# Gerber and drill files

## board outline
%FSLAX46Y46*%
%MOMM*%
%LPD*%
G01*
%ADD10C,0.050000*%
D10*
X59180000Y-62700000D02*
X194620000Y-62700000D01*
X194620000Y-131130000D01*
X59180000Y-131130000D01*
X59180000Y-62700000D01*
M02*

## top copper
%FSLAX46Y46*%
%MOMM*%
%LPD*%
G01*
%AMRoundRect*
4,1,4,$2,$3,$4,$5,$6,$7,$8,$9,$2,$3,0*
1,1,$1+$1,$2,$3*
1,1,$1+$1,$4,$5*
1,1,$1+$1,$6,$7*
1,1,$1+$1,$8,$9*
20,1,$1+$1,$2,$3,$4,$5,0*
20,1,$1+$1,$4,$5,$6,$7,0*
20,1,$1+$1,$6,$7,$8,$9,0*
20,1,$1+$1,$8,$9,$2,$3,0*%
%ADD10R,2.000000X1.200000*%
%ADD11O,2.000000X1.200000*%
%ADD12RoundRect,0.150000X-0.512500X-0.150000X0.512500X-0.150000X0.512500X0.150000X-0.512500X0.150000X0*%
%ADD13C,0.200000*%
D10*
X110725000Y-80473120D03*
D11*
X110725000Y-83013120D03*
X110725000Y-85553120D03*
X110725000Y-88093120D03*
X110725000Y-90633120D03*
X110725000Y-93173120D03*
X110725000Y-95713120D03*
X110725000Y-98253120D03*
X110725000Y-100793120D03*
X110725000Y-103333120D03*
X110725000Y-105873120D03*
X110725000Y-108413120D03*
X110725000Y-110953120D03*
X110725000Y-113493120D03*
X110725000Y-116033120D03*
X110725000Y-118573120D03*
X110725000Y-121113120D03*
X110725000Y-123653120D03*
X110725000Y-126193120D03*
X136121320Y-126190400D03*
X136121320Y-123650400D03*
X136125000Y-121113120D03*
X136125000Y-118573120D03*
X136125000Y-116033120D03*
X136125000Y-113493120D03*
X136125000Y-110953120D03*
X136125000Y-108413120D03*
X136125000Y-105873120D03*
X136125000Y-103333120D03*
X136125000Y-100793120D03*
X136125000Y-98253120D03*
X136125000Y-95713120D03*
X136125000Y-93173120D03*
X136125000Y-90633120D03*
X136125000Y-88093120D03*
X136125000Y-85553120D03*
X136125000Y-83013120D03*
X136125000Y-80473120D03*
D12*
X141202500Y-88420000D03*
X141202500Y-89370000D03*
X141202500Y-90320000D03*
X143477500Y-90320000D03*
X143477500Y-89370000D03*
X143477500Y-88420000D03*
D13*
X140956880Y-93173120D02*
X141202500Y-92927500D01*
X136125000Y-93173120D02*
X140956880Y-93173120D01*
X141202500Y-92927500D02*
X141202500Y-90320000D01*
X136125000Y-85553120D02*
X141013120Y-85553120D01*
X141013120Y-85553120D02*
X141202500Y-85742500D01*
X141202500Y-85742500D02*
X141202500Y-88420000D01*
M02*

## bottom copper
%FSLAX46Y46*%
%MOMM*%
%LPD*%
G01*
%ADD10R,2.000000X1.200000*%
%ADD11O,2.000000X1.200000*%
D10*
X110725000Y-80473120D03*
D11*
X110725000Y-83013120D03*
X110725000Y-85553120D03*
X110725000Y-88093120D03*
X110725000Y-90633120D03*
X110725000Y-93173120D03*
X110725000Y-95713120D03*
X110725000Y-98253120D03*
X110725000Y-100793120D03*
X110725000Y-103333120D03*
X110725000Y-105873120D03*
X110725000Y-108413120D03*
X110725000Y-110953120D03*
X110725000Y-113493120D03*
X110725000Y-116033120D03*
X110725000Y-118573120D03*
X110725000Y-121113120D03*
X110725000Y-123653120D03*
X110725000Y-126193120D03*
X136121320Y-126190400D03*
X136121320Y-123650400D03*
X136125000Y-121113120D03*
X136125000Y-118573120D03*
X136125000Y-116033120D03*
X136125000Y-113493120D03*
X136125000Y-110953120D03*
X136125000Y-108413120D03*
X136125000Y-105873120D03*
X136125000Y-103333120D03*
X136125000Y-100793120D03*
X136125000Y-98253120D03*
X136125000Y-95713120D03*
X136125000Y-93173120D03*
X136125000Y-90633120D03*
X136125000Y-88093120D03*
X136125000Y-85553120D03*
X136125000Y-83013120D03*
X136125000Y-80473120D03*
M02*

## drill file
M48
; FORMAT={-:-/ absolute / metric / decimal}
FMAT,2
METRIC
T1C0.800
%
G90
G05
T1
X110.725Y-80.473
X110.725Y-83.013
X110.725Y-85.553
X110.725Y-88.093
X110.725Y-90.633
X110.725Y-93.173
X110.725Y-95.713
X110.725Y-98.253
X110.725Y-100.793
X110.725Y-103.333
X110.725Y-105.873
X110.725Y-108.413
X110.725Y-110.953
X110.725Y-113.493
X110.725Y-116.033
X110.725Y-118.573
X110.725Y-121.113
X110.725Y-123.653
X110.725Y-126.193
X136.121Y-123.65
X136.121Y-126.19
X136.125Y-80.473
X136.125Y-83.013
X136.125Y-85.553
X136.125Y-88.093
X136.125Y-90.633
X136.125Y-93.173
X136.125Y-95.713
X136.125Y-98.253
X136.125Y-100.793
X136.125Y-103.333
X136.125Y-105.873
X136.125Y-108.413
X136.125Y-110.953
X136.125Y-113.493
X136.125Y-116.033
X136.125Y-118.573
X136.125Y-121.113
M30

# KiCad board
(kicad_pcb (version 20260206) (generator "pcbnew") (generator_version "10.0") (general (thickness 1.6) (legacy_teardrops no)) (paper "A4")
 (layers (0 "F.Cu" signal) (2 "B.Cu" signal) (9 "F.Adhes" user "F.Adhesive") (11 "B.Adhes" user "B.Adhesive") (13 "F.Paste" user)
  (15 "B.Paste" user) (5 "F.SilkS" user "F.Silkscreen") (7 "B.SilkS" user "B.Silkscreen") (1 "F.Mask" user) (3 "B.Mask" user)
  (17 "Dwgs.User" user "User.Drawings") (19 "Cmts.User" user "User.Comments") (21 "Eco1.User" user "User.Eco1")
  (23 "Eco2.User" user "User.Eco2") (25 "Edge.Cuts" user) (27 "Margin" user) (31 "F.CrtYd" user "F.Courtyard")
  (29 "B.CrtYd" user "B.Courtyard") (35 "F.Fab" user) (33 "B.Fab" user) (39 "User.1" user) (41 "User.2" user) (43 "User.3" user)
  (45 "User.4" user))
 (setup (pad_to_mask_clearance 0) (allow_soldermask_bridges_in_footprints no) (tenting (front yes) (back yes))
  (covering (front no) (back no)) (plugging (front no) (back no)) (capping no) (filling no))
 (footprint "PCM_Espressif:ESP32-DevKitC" (layer "F.Cu") (at 110.725 80.47312)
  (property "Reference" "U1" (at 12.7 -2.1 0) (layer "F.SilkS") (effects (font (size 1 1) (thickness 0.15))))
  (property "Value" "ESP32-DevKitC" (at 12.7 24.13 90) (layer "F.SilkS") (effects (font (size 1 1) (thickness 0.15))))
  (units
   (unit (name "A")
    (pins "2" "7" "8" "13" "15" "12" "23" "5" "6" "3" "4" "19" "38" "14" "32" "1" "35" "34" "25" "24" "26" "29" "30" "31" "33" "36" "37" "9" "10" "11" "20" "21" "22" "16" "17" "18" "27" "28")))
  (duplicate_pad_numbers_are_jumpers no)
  (pad "1" thru_hole rect (at 0 0 270) (size 1.2 2) (drill 0.8) (layers "*.Cu" "*.Mask") (remove_unused_layers no) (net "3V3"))
  (pad "2" thru_hole oval (at 0 2.54 270) (size 1.2 2) (drill 0.8) (layers "*.Cu" "*.Mask") (remove_unused_layers no)
   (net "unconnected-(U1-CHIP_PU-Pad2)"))
  (pad "3" thru_hole oval (at 0 5.08 270) (size 1.2 2) (drill 0.8) (layers "*.Cu" "*.Mask") (remove_unused_layers no)
   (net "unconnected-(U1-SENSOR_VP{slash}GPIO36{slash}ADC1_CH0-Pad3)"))
  (pad "4" thru_hole oval (at 0 7.62 270) (size 1.2 2) (drill 0.8) (layers "*.Cu" "*.Mask") (remove_unused_layers no)
   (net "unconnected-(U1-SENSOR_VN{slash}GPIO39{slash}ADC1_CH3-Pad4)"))
  (pad "5" thru_hole oval (at 0 10.16 270) (size 1.2 2) (drill 0.8) (layers "*.Cu" "*.Mask") (remove_unused_layers no)
   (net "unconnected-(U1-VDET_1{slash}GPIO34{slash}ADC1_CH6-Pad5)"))
  (pad "6" thru_hole oval (at 0 12.7 270) (size 1.2 2) (drill 0.8) (layers "*.Cu" "*.Mask") (remove_unused_layers no)
   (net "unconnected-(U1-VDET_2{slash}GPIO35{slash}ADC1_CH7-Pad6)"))
  (pad "7" thru_hole oval (at 0 15.24 270) (size 1.2 2) (drill 0.8) (layers "*.Cu" "*.Mask") (remove_unused_layers no)
   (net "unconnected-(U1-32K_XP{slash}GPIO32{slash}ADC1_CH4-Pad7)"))
  (pad "8" thru_hole oval (at 0 17.78 270) (size 1.2 2) (drill 0.8) (layers "*.Cu" "*.Mask") (remove_unused_layers no)
   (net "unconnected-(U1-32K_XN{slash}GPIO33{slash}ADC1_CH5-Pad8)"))
  (pad "9" thru_hole oval (at 0 20.32 270) (size 1.2 2) (drill 0.8) (layers "*.Cu" "*.Mask") (remove_unused_layers no) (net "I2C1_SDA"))
  (pad "10" thru_hole oval (at 0 22.86 270) (size 1.2 2) (drill 0.8) (layers "*.Cu" "*.Mask") (remove_unused_layers no) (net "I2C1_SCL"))
  (pad "11" thru_hole oval (at 0 25.4 270) (size 1.2 2) (drill 0.8) (layers "*.Cu" "*.Mask") (remove_unused_layers no)
   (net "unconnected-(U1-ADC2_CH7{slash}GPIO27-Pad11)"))
  (pad "12" thru_hole oval (at 0 27.94 270) (size 1.2 2) (drill 0.8) (layers "*.Cu" "*.Mask") (remove_unused_layers no)
   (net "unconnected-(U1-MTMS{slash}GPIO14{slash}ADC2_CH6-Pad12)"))
  (pad "13" thru_hole oval (at 0 30.48 270) (size 1.2 2) (drill 0.8) (layers "*.Cu" "*.Mask") (remove_unused_layers no)
   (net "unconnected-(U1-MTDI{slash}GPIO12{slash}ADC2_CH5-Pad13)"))
  (pad "14" thru_hole oval (at 0 33.02 270) (size 1.2 2) (drill 0.8) (layers "*.Cu" "*.Mask") (remove_unused_layers no) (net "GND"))
  (pad "15" thru_hole oval (at 0 35.56 270) (size 1.2 2) (drill 0.8) (layers "*.Cu" "*.Mask") (remove_unused_layers no)
   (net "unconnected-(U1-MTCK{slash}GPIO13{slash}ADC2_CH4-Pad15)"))
  (pad "16" thru_hole oval (at 0 38.1 270) (size 1.2 2) (drill 0.8) (layers "*.Cu" "*.Mask") (remove_unused_layers no)
   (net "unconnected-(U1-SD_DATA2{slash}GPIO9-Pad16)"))
  (pad "17" thru_hole oval (at 0 40.64 270) (size 1.2 2) (drill 0.8) (layers "*.Cu" "*.Mask") (remove_unused_layers no)
   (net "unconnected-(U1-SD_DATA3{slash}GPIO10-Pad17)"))
  (pad "18" thru_hole oval (at 0 43.18 270) (size 1.2 2) (drill 0.8) (layers "*.Cu" "*.Mask") (remove_unused_layers no)
   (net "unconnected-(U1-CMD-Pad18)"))
  (pad "19" thru_hole oval (at 0 45.72 270) (size 1.2 2) (drill 0.8) (layers "*.Cu" "*.Mask") (remove_unused_layers no) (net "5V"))
  (pad "20" thru_hole oval (at 25.39632 45.71728 270) (size 1.2 2) (drill 0.8) (layers "*.Cu" "*.Mask") (remove_unused_layers no)
   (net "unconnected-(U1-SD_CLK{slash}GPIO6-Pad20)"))
  (pad "21" thru_hole oval (at 25.39632 43.17728 270) (size 1.2 2) (drill 0.8) (layers "*.Cu" "*.Mask") (remove_unused_layers no)
   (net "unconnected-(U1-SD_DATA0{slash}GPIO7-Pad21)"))
  (pad "22" thru_hole oval (at 25.4 40.64 270) (size 1.2 2) (drill 0.8) (layers "*.Cu" "*.Mask") (remove_unused_layers no)
   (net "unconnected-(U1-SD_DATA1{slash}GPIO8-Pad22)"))
  (pad "23" thru_hole oval (at 25.4 38.1 270) (size 1.2 2) (drill 0.8) (layers "*.Cu" "*.Mask") (remove_unused_layers no)
   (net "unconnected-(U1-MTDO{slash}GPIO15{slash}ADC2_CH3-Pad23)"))
  (pad "24" thru_hole oval (at 25.4 35.56 270) (size 1.2 2) (drill 0.8) (layers "*.Cu" "*.Mask") (remove_unused_layers no)
   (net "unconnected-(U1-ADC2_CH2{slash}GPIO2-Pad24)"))
  (pad "25" thru_hole oval (at 25.4 33.02 270) (size 1.2 2) (drill 0.8) (layers "*.Cu" "*.Mask") (remove_unused_layers no)
   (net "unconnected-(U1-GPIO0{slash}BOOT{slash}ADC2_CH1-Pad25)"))
  (pad "26" thru_hole oval (at 25.4 30.48 270) (size 1.2 2) (drill 0.8) (layers "*.Cu" "*.Mask") (remove_unused_layers no)
   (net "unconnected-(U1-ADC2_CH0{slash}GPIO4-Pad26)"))
  (pad "27" thru_hole oval (at 25.4 27.94 270) (size 1.2 2) (drill 0.8) (layers "*.Cu" "*.Mask") (remove_unused_layers no)
   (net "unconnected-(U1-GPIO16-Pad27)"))
  (pad "28" thru_hole oval (at 25.4 25.4 270) (size 1.2 2) (drill 0.8) (layers "*.Cu" "*.Mask") (remove_unused_layers no)
   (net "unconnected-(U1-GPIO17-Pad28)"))
  (pad "29" thru_hole oval (at 25.4 22.86 270) (size 1.2 2) (drill 0.8) (layers "*.Cu" "*.Mask") (remove_unused_layers no)
   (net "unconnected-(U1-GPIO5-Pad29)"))
  (pad "30" thru_hole oval (at 25.4 20.32 270) (size 1.2 2) (drill 0.8) (layers "*.Cu" "*.Mask") (remove_unused_layers no)
   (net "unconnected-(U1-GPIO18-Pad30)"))
  (pad "31" thru_hole oval (at 25.4 17.78 270) (size 1.2 2) (drill 0.8) (layers "*.Cu" "*.Mask") (remove_unused_layers no)
   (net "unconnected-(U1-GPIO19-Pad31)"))
  (pad "32" thru_hole oval (at 25.4 15.24 270) (size 1.2 2) (drill 0.8) (layers "*.Cu" "*.Mask") (remove_unused_layers no) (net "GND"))
  (pad "33" thru_hole oval (at 25.4 12.7 270) (size 1.2 2) (drill 0.8) (layers "*.Cu" "*.Mask") (remove_unused_layers no) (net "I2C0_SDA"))
  (pad "34" thru_hole oval (at 25.4 10.16 270) (size 1.2 2) (drill 0.8) (layers "*.Cu" "*.Mask") (remove_unused_layers no)
   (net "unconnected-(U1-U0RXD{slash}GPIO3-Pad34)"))
  (pad "35" thru_hole oval (at 25.4 7.62 270) (size 1.2 2) (drill 0.8) (layers "*.Cu" "*.Mask") (remove_unused_layers no)
   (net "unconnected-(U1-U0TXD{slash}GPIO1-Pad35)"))
  (pad "36" thru_hole oval (at 25.4 5.08 270) (size 1.2 2) (drill 0.8) (layers "*.Cu" "*.Mask") (remove_unused_layers no) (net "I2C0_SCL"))
  (pad "37" thru_hole oval (at 25.4 2.54 270) (size 1.2 2) (drill 0.8) (layers "*.Cu" "*.Mask") (remove_unused_layers no)
   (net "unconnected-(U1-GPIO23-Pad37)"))
  (pad "38" thru_hole oval (at 25.4 0 270) (size 1.2 2) (drill 0.8) (layers "*.Cu" "*.Mask") (remove_unused_layers no) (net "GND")))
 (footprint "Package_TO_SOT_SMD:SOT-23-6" (layer "F.Cu") (at 142.34 89.37)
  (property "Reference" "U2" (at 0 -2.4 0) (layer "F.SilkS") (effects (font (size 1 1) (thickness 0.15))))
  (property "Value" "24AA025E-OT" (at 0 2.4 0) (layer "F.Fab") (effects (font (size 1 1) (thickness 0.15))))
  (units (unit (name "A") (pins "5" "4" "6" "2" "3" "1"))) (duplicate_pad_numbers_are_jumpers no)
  (pad "1" smd roundrect (at -1.1375 -0.95) (size 1.325 0.6) (layers "F.Cu" "F.Mask" "F.Paste") (roundrect_rratio 0.25) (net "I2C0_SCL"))
  (pad "2" smd roundrect (at -1.1375 0) (size 1.325 0.6) (layers "F.Cu" "F.Mask" "F.Paste") (roundrect_rratio 0.25) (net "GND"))
  (pad "3" smd roundrect (at -1.1375 0.95) (size 1.325 0.6) (layers "F.Cu" "F.Mask" "F.Paste") (roundrect_rratio 0.25) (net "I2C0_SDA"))
  (pad "4" smd roundrect (at 1.1375 0.95) (size 1.325 0.6) (layers "F.Cu" "F.Mask" "F.Paste") (roundrect_rratio 0.25) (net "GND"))
  (pad "5" smd roundrect (at 1.1375 0) (size 1.325 0.6) (layers "F.Cu" "F.Mask" "F.Paste") (roundrect_rratio 0.25) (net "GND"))
  (pad "6" smd roundrect (at 1.1375 -0.95) (size 1.325 0.6) (layers "F.Cu" "F.Mask" "F.Paste") (roundrect_rratio 0.25) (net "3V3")))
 (gr_rect (start 59.18 62.7) (end 194.62 131.13) (stroke (width 0.05) (type default)) (fill no) (layer "Edge.Cuts"))
 (segment (start 140.95688 93.17312) (end 141.2025 92.9275) (width 0.2) (layer "F.Cu") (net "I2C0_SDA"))
 (segment (start 136.125 93.17312) (end 140.95688 93.17312) (width 0.2) (layer "F.Cu") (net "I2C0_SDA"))
 (segment (start 141.2025 92.9275) (end 141.2025 90.32) (width 0.2) (layer "F.Cu") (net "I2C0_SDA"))
 (segment (start 136.125 85.55312) (end 141.01312 85.55312) (width 0.2) (layer "F.Cu") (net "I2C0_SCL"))
 (segment (start 141.01312 85.55312) (end 141.2025 85.7425) (width 0.2) (layer "F.Cu") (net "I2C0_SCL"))
 (segment (start 141.2025 85.7425) (end 141.2025 88.42) (width 0.2) (layer "F.Cu") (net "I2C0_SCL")))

